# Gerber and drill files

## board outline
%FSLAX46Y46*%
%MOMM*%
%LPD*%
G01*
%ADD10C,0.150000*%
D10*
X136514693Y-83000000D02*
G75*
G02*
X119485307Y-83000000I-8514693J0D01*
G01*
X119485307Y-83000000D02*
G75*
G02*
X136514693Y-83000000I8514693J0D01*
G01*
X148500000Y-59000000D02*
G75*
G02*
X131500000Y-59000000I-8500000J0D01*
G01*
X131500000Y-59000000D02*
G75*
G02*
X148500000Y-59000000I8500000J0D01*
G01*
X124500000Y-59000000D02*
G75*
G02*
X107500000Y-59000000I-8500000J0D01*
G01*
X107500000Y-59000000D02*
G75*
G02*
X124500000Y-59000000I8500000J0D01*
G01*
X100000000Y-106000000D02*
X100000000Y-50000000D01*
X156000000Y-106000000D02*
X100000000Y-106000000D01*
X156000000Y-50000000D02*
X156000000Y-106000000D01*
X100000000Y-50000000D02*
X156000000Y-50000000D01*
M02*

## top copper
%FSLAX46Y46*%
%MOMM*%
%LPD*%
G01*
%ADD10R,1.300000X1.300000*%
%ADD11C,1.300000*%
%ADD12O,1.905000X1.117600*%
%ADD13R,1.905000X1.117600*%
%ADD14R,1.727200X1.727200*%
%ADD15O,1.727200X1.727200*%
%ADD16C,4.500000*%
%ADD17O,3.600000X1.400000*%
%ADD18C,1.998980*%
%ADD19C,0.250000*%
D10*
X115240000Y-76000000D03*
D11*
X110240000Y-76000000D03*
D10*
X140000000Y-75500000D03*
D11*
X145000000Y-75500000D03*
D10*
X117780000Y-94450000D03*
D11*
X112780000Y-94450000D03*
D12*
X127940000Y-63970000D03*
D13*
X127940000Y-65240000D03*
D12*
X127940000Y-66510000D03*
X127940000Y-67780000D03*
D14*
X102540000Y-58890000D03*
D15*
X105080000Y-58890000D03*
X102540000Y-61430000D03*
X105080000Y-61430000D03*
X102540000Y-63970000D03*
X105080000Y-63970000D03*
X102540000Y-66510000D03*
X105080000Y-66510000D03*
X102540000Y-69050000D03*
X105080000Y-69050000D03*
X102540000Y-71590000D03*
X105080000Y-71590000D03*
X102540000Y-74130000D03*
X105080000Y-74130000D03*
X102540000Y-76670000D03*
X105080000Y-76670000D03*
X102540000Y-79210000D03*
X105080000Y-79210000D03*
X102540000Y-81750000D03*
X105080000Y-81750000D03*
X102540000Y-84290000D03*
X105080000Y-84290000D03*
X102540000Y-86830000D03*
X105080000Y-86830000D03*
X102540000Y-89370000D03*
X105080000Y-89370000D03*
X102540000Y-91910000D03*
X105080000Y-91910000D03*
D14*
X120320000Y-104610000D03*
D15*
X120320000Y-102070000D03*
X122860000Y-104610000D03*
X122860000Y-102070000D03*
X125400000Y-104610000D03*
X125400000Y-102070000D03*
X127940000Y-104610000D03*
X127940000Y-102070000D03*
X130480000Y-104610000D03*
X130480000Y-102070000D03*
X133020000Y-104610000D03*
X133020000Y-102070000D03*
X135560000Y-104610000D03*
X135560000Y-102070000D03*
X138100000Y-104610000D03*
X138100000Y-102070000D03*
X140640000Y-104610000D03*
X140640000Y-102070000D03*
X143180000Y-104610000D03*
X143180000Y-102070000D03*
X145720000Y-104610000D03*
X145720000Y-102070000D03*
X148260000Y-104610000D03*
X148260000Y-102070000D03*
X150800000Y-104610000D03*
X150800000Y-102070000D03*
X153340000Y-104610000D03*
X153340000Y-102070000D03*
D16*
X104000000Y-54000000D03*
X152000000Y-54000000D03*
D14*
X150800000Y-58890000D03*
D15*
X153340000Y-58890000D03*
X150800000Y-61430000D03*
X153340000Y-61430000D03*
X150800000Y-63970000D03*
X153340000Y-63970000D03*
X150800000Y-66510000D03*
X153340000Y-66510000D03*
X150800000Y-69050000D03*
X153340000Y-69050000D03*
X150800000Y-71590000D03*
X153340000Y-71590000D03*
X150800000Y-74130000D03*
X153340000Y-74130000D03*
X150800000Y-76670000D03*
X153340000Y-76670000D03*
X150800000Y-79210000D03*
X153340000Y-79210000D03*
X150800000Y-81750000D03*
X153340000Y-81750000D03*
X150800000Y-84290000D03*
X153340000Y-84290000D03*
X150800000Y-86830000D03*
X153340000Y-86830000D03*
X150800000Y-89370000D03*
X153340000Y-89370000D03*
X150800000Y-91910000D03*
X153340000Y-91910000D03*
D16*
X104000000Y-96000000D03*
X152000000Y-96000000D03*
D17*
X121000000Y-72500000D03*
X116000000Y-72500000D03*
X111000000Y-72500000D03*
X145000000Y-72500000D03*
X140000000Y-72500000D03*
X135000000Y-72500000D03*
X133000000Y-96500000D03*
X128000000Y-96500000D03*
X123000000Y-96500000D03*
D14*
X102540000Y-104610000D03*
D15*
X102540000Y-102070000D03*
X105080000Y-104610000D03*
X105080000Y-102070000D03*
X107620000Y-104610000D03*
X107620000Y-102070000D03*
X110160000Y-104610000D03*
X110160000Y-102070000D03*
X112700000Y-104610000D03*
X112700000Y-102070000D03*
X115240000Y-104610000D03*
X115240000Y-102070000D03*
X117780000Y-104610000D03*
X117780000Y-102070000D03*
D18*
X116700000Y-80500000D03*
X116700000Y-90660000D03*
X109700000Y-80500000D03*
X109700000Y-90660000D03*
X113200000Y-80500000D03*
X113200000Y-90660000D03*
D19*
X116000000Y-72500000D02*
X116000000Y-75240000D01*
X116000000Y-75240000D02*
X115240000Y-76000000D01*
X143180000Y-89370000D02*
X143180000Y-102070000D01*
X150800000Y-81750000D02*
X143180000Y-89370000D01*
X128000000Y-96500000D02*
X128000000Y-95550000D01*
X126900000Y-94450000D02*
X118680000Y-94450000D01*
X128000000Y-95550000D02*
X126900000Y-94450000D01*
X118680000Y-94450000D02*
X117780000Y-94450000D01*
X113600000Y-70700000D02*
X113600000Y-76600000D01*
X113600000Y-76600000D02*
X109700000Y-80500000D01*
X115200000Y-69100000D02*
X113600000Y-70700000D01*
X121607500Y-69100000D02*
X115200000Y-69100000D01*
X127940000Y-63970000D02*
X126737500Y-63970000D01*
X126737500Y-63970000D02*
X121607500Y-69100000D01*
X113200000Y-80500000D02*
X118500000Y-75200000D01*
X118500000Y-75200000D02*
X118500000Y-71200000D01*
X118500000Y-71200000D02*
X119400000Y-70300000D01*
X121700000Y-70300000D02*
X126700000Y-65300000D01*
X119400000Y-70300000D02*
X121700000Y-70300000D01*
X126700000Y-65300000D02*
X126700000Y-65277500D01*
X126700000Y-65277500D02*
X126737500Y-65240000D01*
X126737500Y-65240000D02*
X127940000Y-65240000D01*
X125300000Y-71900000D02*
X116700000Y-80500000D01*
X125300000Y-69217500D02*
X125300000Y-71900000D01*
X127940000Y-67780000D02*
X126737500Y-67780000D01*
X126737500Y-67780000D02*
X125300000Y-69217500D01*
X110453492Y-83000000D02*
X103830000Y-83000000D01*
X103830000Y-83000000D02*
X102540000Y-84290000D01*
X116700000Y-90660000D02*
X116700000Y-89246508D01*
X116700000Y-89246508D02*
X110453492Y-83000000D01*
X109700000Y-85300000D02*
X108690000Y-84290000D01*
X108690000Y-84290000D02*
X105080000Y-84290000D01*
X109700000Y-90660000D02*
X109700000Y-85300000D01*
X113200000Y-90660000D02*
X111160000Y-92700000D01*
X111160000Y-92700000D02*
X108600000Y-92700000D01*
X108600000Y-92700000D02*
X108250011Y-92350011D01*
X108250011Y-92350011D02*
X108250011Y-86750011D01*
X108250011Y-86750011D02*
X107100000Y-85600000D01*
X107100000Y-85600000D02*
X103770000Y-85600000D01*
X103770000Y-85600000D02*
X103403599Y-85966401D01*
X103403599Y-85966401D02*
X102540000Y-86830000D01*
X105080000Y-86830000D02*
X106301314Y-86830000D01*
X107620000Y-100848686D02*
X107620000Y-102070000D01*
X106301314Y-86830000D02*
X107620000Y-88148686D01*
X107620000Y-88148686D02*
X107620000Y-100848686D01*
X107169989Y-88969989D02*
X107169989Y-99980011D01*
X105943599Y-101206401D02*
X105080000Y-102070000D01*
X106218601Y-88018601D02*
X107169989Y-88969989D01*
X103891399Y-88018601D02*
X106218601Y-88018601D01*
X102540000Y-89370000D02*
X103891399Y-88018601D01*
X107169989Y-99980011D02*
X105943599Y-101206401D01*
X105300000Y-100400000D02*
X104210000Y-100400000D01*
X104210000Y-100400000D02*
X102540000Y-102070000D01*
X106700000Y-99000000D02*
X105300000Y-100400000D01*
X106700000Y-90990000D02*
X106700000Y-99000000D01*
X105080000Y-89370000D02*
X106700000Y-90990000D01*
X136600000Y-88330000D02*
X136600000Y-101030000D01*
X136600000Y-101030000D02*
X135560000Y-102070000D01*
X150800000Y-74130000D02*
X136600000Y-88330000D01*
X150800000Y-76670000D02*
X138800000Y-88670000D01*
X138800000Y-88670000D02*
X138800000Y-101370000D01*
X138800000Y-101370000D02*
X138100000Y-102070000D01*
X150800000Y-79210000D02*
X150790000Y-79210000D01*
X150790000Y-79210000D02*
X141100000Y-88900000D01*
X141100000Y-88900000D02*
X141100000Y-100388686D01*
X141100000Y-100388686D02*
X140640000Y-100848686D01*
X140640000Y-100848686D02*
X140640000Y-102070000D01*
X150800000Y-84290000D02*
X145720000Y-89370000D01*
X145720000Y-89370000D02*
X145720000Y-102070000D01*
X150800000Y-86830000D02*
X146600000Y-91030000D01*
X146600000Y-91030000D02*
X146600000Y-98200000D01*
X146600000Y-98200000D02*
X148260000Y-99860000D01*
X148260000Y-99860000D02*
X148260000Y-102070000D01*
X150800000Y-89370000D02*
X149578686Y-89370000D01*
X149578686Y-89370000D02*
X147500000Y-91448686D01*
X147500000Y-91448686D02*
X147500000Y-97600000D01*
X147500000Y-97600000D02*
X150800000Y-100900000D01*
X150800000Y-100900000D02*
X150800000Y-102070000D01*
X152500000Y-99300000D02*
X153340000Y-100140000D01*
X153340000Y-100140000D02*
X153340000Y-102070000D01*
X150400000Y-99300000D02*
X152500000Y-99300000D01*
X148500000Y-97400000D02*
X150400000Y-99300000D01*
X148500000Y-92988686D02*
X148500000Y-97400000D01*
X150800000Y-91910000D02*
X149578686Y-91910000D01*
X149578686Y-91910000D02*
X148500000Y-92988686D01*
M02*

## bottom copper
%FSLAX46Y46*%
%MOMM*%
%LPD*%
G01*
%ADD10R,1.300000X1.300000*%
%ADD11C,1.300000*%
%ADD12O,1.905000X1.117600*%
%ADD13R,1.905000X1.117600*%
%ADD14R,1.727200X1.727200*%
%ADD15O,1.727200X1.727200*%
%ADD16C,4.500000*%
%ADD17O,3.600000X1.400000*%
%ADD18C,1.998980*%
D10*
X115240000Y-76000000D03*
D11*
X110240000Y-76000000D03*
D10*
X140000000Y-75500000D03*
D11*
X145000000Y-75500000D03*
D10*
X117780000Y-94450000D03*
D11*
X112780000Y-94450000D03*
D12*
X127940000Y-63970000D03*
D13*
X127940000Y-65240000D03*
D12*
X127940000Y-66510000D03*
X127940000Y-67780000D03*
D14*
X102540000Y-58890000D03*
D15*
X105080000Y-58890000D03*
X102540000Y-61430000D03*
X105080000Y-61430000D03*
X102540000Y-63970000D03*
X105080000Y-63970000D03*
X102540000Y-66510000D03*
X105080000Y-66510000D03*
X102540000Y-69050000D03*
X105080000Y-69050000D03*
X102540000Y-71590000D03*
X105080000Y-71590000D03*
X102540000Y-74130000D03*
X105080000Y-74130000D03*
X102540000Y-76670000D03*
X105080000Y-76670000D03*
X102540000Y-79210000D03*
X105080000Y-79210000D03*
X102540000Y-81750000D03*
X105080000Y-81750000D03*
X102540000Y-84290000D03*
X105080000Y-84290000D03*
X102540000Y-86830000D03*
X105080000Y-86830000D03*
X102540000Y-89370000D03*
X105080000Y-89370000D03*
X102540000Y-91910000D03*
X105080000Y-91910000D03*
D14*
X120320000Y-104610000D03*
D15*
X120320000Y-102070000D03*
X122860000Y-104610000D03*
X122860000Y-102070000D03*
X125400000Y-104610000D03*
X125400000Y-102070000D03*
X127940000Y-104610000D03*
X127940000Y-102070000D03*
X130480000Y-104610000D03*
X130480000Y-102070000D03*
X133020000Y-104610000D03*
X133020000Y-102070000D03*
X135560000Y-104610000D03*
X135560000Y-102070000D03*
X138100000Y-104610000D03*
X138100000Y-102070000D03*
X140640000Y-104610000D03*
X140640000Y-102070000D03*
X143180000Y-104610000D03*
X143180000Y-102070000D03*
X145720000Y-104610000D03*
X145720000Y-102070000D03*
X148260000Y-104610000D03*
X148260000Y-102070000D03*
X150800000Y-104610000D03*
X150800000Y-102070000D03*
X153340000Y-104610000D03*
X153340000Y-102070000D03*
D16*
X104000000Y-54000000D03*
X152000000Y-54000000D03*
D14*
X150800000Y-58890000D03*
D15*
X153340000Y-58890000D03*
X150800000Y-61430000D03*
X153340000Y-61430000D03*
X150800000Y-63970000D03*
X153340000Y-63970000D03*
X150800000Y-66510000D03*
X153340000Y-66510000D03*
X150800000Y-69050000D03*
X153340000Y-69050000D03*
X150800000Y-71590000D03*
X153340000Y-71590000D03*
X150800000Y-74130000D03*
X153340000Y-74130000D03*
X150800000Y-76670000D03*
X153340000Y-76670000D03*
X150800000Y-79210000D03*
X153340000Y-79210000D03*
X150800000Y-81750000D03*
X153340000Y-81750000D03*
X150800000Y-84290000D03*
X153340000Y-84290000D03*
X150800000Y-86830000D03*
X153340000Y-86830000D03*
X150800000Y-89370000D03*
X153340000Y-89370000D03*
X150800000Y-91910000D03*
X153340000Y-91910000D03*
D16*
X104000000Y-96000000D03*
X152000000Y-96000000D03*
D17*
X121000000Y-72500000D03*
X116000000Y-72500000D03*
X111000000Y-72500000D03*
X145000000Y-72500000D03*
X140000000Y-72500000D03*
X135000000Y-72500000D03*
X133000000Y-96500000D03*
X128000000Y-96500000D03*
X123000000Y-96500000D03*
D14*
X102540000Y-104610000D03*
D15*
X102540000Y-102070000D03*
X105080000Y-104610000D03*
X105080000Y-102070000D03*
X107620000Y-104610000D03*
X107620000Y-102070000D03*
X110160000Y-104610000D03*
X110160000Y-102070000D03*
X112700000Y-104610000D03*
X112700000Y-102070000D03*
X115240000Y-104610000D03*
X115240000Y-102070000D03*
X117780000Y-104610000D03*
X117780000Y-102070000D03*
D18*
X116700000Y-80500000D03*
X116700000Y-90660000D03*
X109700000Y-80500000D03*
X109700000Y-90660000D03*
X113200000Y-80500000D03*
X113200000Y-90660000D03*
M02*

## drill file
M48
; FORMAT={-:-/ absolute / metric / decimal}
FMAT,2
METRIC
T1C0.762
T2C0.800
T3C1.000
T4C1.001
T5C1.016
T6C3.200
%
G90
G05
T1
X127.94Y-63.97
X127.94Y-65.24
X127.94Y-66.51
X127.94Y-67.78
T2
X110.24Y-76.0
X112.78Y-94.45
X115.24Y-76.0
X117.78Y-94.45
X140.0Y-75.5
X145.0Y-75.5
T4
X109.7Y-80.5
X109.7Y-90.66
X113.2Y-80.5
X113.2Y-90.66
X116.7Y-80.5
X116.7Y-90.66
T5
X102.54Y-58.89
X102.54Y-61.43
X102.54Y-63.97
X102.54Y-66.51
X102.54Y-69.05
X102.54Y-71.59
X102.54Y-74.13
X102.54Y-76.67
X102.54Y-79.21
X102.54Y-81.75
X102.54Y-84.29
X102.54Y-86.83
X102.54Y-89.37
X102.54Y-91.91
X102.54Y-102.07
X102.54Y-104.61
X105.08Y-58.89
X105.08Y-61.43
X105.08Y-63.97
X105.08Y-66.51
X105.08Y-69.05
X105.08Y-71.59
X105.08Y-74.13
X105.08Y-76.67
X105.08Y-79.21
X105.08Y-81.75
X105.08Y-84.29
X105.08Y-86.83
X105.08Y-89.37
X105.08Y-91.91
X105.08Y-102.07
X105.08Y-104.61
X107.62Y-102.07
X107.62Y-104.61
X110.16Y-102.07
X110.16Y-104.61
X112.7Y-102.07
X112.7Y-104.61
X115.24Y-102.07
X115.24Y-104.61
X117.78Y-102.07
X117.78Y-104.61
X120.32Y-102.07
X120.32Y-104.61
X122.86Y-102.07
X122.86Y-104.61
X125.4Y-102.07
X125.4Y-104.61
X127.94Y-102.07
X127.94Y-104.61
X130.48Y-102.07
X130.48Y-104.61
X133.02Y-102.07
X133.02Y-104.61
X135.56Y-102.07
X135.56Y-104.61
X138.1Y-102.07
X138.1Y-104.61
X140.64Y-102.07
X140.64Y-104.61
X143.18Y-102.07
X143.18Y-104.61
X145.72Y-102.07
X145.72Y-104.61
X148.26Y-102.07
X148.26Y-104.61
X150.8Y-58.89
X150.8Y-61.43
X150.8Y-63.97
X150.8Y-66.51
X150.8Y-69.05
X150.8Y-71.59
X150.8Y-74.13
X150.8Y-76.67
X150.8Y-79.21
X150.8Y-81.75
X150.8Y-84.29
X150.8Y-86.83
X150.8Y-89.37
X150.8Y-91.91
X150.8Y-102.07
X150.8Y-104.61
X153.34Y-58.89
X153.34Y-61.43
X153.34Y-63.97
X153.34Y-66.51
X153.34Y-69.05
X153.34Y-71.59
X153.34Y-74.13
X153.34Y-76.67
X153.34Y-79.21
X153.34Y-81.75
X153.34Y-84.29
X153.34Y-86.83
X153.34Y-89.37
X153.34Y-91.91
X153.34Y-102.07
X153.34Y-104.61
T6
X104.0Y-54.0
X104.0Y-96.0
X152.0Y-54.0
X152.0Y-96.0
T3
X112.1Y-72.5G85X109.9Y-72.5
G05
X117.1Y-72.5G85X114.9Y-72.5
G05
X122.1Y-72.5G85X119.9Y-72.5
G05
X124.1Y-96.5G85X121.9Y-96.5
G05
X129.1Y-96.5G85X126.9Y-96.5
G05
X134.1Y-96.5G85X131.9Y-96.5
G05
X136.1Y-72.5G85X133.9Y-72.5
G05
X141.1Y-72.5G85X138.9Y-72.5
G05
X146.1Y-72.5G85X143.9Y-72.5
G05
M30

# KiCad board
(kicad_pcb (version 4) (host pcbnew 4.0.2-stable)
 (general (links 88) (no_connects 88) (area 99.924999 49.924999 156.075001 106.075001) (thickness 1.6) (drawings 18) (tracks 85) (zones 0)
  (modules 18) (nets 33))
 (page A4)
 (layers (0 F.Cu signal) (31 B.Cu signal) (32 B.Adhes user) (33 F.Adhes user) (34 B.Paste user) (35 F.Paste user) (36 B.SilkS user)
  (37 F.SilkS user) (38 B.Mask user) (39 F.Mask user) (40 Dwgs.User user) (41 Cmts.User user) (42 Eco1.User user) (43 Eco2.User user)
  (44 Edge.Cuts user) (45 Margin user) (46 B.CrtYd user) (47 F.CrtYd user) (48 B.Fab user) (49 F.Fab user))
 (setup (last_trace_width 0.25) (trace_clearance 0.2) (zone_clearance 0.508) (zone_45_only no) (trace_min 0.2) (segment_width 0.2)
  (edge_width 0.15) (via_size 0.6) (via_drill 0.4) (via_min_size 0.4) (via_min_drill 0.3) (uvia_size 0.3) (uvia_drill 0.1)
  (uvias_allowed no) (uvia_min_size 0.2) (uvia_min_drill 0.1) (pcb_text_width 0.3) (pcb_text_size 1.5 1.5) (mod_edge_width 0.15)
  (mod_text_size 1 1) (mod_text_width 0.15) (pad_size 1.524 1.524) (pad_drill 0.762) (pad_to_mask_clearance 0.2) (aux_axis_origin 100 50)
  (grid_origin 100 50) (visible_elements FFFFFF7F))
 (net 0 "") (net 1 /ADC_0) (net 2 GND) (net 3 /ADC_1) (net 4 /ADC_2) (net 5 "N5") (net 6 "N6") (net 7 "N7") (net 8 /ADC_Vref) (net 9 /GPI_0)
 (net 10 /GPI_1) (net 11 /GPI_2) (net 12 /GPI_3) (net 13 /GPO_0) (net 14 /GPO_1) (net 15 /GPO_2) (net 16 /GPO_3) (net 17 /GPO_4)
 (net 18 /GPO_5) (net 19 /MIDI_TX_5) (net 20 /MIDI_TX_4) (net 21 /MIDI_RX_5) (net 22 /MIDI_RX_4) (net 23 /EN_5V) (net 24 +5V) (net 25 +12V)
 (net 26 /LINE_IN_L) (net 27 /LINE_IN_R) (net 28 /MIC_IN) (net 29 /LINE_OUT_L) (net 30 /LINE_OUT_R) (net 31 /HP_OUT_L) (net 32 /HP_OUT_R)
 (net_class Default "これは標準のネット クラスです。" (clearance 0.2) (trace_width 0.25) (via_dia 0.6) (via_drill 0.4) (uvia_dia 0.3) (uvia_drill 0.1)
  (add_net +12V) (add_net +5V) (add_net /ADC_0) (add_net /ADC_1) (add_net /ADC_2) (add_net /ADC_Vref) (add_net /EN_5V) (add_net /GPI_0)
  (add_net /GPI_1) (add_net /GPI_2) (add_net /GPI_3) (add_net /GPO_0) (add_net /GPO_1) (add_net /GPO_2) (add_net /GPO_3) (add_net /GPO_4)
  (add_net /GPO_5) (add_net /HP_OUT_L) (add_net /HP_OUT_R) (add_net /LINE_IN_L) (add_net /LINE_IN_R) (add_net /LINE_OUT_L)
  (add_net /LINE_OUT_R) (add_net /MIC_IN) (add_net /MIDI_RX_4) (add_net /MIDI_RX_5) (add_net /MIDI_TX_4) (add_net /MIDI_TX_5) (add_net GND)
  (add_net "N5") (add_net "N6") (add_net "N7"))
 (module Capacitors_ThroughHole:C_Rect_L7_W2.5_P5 (layer F.Cu) (at 115.24 76 180)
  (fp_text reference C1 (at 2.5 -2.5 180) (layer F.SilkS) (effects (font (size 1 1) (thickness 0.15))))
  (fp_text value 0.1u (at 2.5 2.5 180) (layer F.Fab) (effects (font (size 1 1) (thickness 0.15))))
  (pad 1 thru_hole rect (at 0 0 180) (size 1.3 1.3) (drill 0.8) (layers *.Cu *.Mask) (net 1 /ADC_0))
  (pad 2 thru_hole circle (at 5 0 180) (size 1.3 1.3) (drill 0.8) (layers *.Cu *.Mask) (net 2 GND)))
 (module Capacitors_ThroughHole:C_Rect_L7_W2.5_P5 (layer F.Cu) (at 140 75.5)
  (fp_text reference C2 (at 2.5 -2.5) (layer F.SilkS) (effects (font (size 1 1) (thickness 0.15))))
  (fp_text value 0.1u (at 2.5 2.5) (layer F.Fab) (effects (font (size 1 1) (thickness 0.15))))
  (pad 1 thru_hole rect (at 0 0) (size 1.3 1.3) (drill 0.8) (layers *.Cu *.Mask) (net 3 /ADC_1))
  (pad 2 thru_hole circle (at 5 0) (size 1.3 1.3) (drill 0.8) (layers *.Cu *.Mask) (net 2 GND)))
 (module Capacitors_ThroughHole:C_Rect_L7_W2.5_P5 (layer F.Cu) (at 117.78 94.45 180)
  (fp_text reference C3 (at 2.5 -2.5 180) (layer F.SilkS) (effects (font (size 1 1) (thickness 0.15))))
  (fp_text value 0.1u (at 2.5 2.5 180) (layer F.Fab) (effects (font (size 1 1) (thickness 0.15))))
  (pad 1 thru_hole rect (at 0 0 180) (size 1.3 1.3) (drill 0.8) (layers *.Cu *.Mask) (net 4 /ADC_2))
  (pad 2 thru_hole circle (at 5 0 180) (size 1.3 1.3) (drill 0.8) (layers *.Cu *.Mask) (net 2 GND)))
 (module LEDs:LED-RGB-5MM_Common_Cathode (layer B.Cu) (at 127.94 63.97 180)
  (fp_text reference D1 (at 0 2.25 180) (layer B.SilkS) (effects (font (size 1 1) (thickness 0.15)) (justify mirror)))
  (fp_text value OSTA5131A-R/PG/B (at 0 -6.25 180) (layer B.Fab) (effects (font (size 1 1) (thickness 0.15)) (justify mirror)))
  (pad 1 thru_hole oval (at 0 0 180) (size 1.905 1.1176) (drill 0.762) (layers *.Cu *.Mask) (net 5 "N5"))
  (pad 2 thru_hole rect (at 0 -1.27 180) (size 1.905 1.1176) (drill 0.762) (layers *.Cu *.Mask) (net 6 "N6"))
  (pad 3 thru_hole oval (at 0 -2.54 180) (size 1.905 1.1176) (drill 0.762) (layers *.Cu *.Mask) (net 2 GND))
  (pad 4 thru_hole oval (at 0 -3.81 180) (size 1.905 1.1176) (drill 0.762) (layers *.Cu *.Mask) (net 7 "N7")))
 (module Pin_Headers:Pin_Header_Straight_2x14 (layer F.Cu) (at 102.54 58.89)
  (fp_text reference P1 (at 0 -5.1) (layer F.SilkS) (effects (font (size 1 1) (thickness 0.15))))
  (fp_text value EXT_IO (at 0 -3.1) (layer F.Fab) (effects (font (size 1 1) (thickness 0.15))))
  (pad 1 thru_hole rect (at 0 0) (size 1.7272 1.7272) (drill 1.016) (layers *.Cu *.Mask) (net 1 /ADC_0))
  (pad 2 thru_hole oval (at 2.54 0) (size 1.7272 1.7272) (drill 1.016) (layers *.Cu *.Mask) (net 3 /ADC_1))
  (pad 3 thru_hole oval (at 0 2.54) (size 1.7272 1.7272) (drill 1.016) (layers *.Cu *.Mask) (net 4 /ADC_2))
  (pad 4 thru_hole oval (at 2.54 2.54) (size 1.7272 1.7272) (drill 1.016) (layers *.Cu *.Mask) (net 2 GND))
  (pad 5 thru_hole oval (at 0 5.08) (size 1.7272 1.7272) (drill 1.016) (layers *.Cu *.Mask) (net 2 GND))
  (pad 6 thru_hole oval (at 2.54 5.08) (size 1.7272 1.7272) (drill 1.016) (layers *.Cu *.Mask) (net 2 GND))
  (pad 7 thru_hole oval (at 0 7.62) (size 1.7272 1.7272) (drill 1.016) (layers *.Cu *.Mask) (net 2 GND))
  (pad 8 thru_hole oval (at 2.54 7.62) (size 1.7272 1.7272) (drill 1.016) (layers *.Cu *.Mask) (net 2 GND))
  (pad 9 thru_hole oval (at 0 10.16) (size 1.7272 1.7272) (drill 1.016) (layers *.Cu *.Mask))
  (pad 10 thru_hole oval (at 2.54 10.16) (size 1.7272 1.7272) (drill 1.016) (layers *.Cu *.Mask) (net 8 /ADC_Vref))
  (pad 11 thru_hole oval (at 0 12.7) (size 1.7272 1.7272) (drill 1.016) (layers *.Cu *.Mask) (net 2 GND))
  (pad 12 thru_hole oval (at 2.54 12.7) (size 1.7272 1.7272) (drill 1.016) (layers *.Cu *.Mask) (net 2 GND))
  (pad 13 thru_hole oval (at 0 15.24) (size 1.7272 1.7272) (drill 1.016) (layers *.Cu *.Mask) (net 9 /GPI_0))
  (pad 14 thru_hole oval (at 2.54 15.24) (size 1.7272 1.7272) (drill 1.016) (layers *.Cu *.Mask) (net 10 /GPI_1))
  (pad 15 thru_hole oval (at 0 17.78) (size 1.7272 1.7272) (drill 1.016) (layers *.Cu *.Mask) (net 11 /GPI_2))
  (pad 16 thru_hole oval (at 2.54 17.78) (size 1.7272 1.7272) (drill 1.016) (layers *.Cu *.Mask) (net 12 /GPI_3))
  (pad 17 thru_hole oval (at 0 20.32) (size 1.7272 1.7272) (drill 1.016) (layers *.Cu *.Mask))
  (pad 18 thru_hole oval (at 2.54 20.32) (size 1.7272 1.7272) (drill 1.016) (layers *.Cu *.Mask))
  (pad 19 thru_hole oval (at 0 22.86) (size 1.7272 1.7272) (drill 1.016) (layers *.Cu *.Mask))
  (pad 20 thru_hole oval (at 2.54 22.86) (size 1.7272 1.7272) (drill 1.016) (layers *.Cu *.Mask))
  (pad 21 thru_hole oval (at 0 25.4) (size 1.7272 1.7272) (drill 1.016) (layers *.Cu *.Mask) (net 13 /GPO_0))
  (pad 22 thru_hole oval (at 2.54 25.4) (size 1.7272 1.7272) (drill 1.016) (layers *.Cu *.Mask) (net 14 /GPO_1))
  (pad 23 thru_hole oval (at 0 27.94) (size 1.7272 1.7272) (drill 1.016) (layers *.Cu *.Mask) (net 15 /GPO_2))
  (pad 24 thru_hole oval (at 2.54 27.94) (size 1.7272 1.7272) (drill 1.016) (layers *.Cu *.Mask) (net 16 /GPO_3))
  (pad 25 thru_hole oval (at 0 30.48) (size 1.7272 1.7272) (drill 1.016) (layers *.Cu *.Mask) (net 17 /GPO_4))
  (pad 26 thru_hole oval (at 2.54 30.48) (size 1.7272 1.7272) (drill 1.016) (layers *.Cu *.Mask) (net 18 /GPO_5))
  (pad 27 thru_hole oval (at 0 33.02) (size 1.7272 1.7272) (drill 1.016) (layers *.Cu *.Mask))
  (pad 28 thru_hole oval (at 2.54 33.02) (size 1.7272 1.7272) (drill 1.016) (layers *.Cu *.Mask)))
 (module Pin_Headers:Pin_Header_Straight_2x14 (layer F.Cu) (at 120.32 104.61 90)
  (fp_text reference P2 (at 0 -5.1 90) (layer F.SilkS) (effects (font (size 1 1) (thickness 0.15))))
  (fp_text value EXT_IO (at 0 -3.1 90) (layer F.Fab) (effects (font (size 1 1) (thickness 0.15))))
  (pad 1 thru_hole rect (at 0 0 90) (size 1.7272 1.7272) (drill 1.016) (layers *.Cu *.Mask) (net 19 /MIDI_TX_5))
  (pad 2 thru_hole oval (at 2.54 0 90) (size 1.7272 1.7272) (drill 1.016) (layers *.Cu *.Mask) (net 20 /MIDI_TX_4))
  (pad 3 thru_hole oval (at 0 2.54 90) (size 1.7272 1.7272) (drill 1.016) (layers *.Cu *.Mask) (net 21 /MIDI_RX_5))
  (pad 4 thru_hole oval (at 2.54 2.54 90) (size 1.7272 1.7272) (drill 1.016) (layers *.Cu *.Mask) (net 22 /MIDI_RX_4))
  (pad 5 thru_hole oval (at 0 5.08 90) (size 1.7272 1.7272) (drill 1.016) (layers *.Cu *.Mask) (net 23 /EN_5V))
  (pad 6 thru_hole oval (at 2.54 5.08 90) (size 1.7272 1.7272) (drill 1.016) (layers *.Cu *.Mask) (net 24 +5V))
  (pad 7 thru_hole oval (at 0 7.62 90) (size 1.7272 1.7272) (drill 1.016) (layers *.Cu *.Mask) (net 2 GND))
  (pad 8 thru_hole oval (at 2.54 7.62 90) (size 1.7272 1.7272) (drill 1.016) (layers *.Cu *.Mask) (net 2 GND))
  (pad 9 thru_hole oval (at 0 10.16 90) (size 1.7272 1.7272) (drill 1.016) (layers *.Cu *.Mask) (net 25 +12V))
  (pad 10 thru_hole oval (at 2.54 10.16 90) (size 1.7272 1.7272) (drill 1.016) (layers *.Cu *.Mask) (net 25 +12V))
  (pad 11 thru_hole oval (at 0 12.7 90) (size 1.7272 1.7272) (drill 1.016) (layers *.Cu *.Mask) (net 2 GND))
  (pad 12 thru_hole oval (at 2.54 12.7 90) (size 1.7272 1.7272) (drill 1.016) (layers *.Cu *.Mask) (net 2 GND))
  (pad 13 thru_hole oval (at 0 15.24 90) (size 1.7272 1.7272) (drill 1.016) (layers *.Cu *.Mask) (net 2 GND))
  (pad 14 thru_hole oval (at 2.54 15.24 90) (size 1.7272 1.7272) (drill 1.016) (layers *.Cu *.Mask) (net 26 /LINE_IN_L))
  (pad 15 thru_hole oval (at 0 17.78 90) (size 1.7272 1.7272) (drill 1.016) (layers *.Cu *.Mask) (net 2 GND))
  (pad 16 thru_hole oval (at 2.54 17.78 90) (size 1.7272 1.7272) (drill 1.016) (layers *.Cu *.Mask) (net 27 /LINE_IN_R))
  (pad 17 thru_hole oval (at 0 20.32 90) (size 1.7272 1.7272) (drill 1.016) (layers *.Cu *.Mask) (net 2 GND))
  (pad 18 thru_hole oval (at 2.54 20.32 90) (size 1.7272 1.7272) (drill 1.016) (layers *.Cu *.Mask) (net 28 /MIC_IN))
  (pad 19 thru_hole oval (at 0 22.86 90) (size 1.7272 1.7272) (drill 1.016) (layers *.Cu *.Mask) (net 2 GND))
  (pad 20 thru_hole oval (at 2.54 22.86 90) (size 1.7272 1.7272) (drill 1.016) (layers *.Cu *.Mask) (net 2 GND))
  (pad 21 thru_hole oval (at 0 25.4 90) (size 1.7272 1.7272) (drill 1.016) (layers *.Cu *.Mask) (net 2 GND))
  (pad 22 thru_hole oval (at 2.54 25.4 90) (size 1.7272 1.7272) (drill 1.016) (layers *.Cu *.Mask) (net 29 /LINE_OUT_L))
  (pad 23 thru_hole oval (at 0 27.94 90) (size 1.7272 1.7272) (drill 1.016) (layers *.Cu *.Mask) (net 2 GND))
  (pad 24 thru_hole oval (at 2.54 27.94 90) (size 1.7272 1.7272) (drill 1.016) (layers *.Cu *.Mask) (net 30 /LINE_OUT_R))
  (pad 25 thru_hole oval (at 0 30.48 90) (size 1.7272 1.7272) (drill 1.016) (layers *.Cu *.Mask) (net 2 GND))
  (pad 26 thru_hole oval (at 2.54 30.48 90) (size 1.7272 1.7272) (drill 1.016) (layers *.Cu *.Mask) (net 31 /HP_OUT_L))
  (pad 27 thru_hole oval (at 0 33.02 90) (size 1.7272 1.7272) (drill 1.016) (layers *.Cu *.Mask) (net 2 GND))
  (pad 28 thru_hole oval (at 2.54 33.02 90) (size 1.7272 1.7272) (drill 1.016) (layers *.Cu *.Mask) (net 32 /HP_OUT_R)))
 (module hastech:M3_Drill (layer F.Cu) (at 104 54)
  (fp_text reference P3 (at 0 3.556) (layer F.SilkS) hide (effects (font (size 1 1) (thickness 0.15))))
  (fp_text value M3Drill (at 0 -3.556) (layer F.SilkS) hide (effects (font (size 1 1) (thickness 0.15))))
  (pad 1 thru_hole circle (at 0 0) (size 4.5 4.5) (drill 3.2) (layers *.Cu *.Mask F.SilkS) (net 2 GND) (zone_connect 2)))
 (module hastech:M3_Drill (layer F.Cu) (at 152 54)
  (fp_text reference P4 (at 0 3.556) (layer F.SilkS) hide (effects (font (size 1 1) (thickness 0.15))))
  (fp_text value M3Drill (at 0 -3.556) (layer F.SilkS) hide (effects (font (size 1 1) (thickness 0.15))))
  (pad 1 thru_hole circle (at 0 0) (size 4.5 4.5) (drill 3.2) (layers *.Cu *.Mask F.SilkS) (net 2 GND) (zone_connect 2)))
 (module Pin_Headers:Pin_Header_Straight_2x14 (layer F.Cu) (at 150.8 58.89)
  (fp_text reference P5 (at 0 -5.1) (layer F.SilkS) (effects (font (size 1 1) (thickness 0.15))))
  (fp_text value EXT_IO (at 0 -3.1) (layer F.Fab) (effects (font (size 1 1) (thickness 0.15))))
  (pad 1 thru_hole rect (at 0 0) (size 1.7272 1.7272) (drill 1.016) (layers *.Cu *.Mask) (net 20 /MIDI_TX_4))
  (pad 2 thru_hole oval (at 2.54 0) (size 1.7272 1.7272) (drill 1.016) (layers *.Cu *.Mask) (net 19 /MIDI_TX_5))
  (pad 3 thru_hole oval (at 0 2.54) (size 1.7272 1.7272) (drill 1.016) (layers *.Cu *.Mask) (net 22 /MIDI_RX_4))
  (pad 4 thru_hole oval (at 2.54 2.54) (size 1.7272 1.7272) (drill 1.016) (layers *.Cu *.Mask) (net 21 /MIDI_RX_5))
  (pad 5 thru_hole oval (at 0 5.08) (size 1.7272 1.7272) (drill 1.016) (layers *.Cu *.Mask) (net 24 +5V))
  (pad 6 thru_hole oval (at 2.54 5.08) (size 1.7272 1.7272) (drill 1.016) (layers *.Cu *.Mask) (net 23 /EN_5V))
  (pad 7 thru_hole oval (at 0 7.62) (size 1.7272 1.7272) (drill 1.016) (layers *.Cu *.Mask) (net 2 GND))
  (pad 8 thru_hole oval (at 2.54 7.62) (size 1.7272 1.7272) (drill 1.016) (layers *.Cu *.Mask) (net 2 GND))
  (pad 9 thru_hole oval (at 0 10.16) (size 1.7272 1.7272) (drill 1.016) (layers *.Cu *.Mask) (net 25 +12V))
  (pad 10 thru_hole oval (at 2.54 10.16) (size 1.7272 1.7272) (drill 1.016) (layers *.Cu *.Mask) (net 25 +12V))
  (pad 11 thru_hole oval (at 0 12.7) (size 1.7272 1.7272) (drill 1.016) (layers *.Cu *.Mask) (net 2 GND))
  (pad 12 thru_hole oval (at 2.54 12.7) (size 1.7272 1.7272) (drill 1.016) (layers *.Cu *.Mask) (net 2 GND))
  (pad 13 thru_hole oval (at 0 15.24) (size 1.7272 1.7272) (drill 1.016) (layers *.Cu *.Mask) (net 26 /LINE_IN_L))
  (pad 14 thru_hole oval (at 2.54 15.24) (size 1.7272 1.7272) (drill 1.016) (layers *.Cu *.Mask) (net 2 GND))
  (pad 15 thru_hole oval (at 0 17.78) (size 1.7272 1.7272) (drill 1.016) (layers *.Cu *.Mask) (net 27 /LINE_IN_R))
  (pad 16 thru_hole oval (at 2.54 17.78) (size 1.7272 1.7272) (drill 1.016) (layers *.Cu *.Mask) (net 2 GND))
  (pad 17 thru_hole oval (at 0 20.32) (size 1.7272 1.7272) (drill 1.016) (layers *.Cu *.Mask) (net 28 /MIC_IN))
  (pad 18 thru_hole oval (at 2.54 20.32) (size 1.7272 1.7272) (drill 1.016) (layers *.Cu *.Mask) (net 2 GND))
  (pad 19 thru_hole oval (at 0 22.86) (size 1.7272 1.7272) (drill 1.016) (layers *.Cu *.Mask) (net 2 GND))
  (pad 20 thru_hole oval (at 2.54 22.86) (size 1.7272 1.7272) (drill 1.016) (layers *.Cu *.Mask) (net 2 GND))
  (pad 21 thru_hole oval (at 0 25.4) (size 1.7272 1.7272) (drill 1.016) (layers *.Cu *.Mask) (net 29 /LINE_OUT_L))
  (pad 22 thru_hole oval (at 2.54 25.4) (size 1.7272 1.7272) (drill 1.016) (layers *.Cu *.Mask) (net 2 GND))
  (pad 23 thru_hole oval (at 0 27.94) (size 1.7272 1.7272) (drill 1.016) (layers *.Cu *.Mask) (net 30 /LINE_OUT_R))
  (pad 24 thru_hole oval (at 2.54 27.94) (size 1.7272 1.7272) (drill 1.016) (layers *.Cu *.Mask) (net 2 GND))
  (pad 25 thru_hole oval (at 0 30.48) (size 1.7272 1.7272) (drill 1.016) (layers *.Cu *.Mask) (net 31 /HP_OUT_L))
  (pad 26 thru_hole oval (at 2.54 30.48) (size 1.7272 1.7272) (drill 1.016) (layers *.Cu *.Mask) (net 2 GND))
  (pad 27 thru_hole oval (at 0 33.02) (size 1.7272 1.7272) (drill 1.016) (layers *.Cu *.Mask) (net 32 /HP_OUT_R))
  (pad 28 thru_hole oval (at 2.54 33.02) (size 1.7272 1.7272) (drill 1.016) (layers *.Cu *.Mask) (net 2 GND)))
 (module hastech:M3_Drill (layer F.Cu) (at 104 96)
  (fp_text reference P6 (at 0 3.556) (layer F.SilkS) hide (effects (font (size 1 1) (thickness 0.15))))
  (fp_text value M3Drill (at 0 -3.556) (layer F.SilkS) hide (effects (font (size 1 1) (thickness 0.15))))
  (pad 1 thru_hole circle (at 0 0) (size 4.5 4.5) (drill 3.2) (layers *.Cu *.Mask F.SilkS) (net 2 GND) (zone_connect 2)))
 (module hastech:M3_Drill (layer F.Cu) (at 152 96)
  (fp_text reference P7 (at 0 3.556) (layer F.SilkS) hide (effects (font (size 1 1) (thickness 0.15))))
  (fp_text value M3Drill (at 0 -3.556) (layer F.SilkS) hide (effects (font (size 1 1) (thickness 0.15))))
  (pad 1 thru_hole circle (at 0 0) (size 4.5 4.5) (drill 3.2) (layers *.Cu *.Mask F.SilkS) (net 2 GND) (zone_connect 2)))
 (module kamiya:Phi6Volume (layer B.Cu) (at 116 59 180)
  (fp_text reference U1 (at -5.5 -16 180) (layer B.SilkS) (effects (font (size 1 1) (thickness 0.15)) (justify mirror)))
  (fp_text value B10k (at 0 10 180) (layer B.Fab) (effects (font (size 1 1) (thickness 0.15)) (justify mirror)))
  (pad 1 thru_hole oval (at -5 -13.5 180) (size 3.6 1.4) (drill oval 3.2 1) (layers *.Cu *.Mask B.SilkS) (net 8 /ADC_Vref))
  (pad 2 thru_hole oval (at 0 -13.5 180) (size 3.6 1.4) (drill oval 3.2 1) (layers *.Cu *.Mask B.SilkS) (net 1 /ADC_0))
  (pad 3 thru_hole oval (at 5 -13.5 180) (size 3.6 1.4) (drill oval 3.2 1) (layers *.Cu *.Mask B.SilkS) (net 2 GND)))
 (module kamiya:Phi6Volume (layer B.Cu) (at 140 59 180)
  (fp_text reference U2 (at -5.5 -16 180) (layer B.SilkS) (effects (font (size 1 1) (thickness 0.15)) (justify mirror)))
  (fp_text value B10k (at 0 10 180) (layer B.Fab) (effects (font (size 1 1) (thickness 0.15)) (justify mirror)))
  (pad 1 thru_hole oval (at -5 -13.5 180) (size 3.6 1.4) (drill oval 3.2 1) (layers *.Cu *.Mask B.SilkS) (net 8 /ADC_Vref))
  (pad 2 thru_hole oval (at 0 -13.5 180) (size 3.6 1.4) (drill oval 3.2 1) (layers *.Cu *.Mask B.SilkS) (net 3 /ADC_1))
  (pad 3 thru_hole oval (at 5 -13.5 180) (size 3.6 1.4) (drill oval 3.2 1) (layers *.Cu *.Mask B.SilkS) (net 2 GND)))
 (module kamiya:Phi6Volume (layer B.Cu) (at 128 83 180)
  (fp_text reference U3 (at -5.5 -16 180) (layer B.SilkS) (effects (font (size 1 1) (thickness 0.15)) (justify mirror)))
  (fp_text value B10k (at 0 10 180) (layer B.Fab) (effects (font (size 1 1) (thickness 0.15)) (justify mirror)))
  (pad 1 thru_hole oval (at -5 -13.5 180) (size 3.6 1.4) (drill oval 3.2 1) (layers *.Cu *.Mask B.SilkS) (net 8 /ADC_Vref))
  (pad 2 thru_hole oval (at 0 -13.5 180) (size 3.6 1.4) (drill oval 3.2 1) (layers *.Cu *.Mask B.SilkS) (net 4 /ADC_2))
  (pad 3 thru_hole oval (at 5 -13.5 180) (size 3.6 1.4) (drill oval 3.2 1) (layers *.Cu *.Mask B.SilkS) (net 2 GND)))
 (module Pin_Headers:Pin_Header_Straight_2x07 (layer F.Cu) (at 102.54 104.61 90)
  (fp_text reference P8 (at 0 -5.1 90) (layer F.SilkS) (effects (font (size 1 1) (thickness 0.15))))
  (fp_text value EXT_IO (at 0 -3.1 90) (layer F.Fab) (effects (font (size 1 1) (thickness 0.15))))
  (pad 1 thru_hole rect (at 0 0 90) (size 1.7272 1.7272) (drill 1.016) (layers *.Cu *.Mask) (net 2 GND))
  (pad 2 thru_hole oval (at 2.54 0 90) (size 1.7272 1.7272) (drill 1.016) (layers *.Cu *.Mask) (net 18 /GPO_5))
  (pad 3 thru_hole oval (at 0 2.54 90) (size 1.7272 1.7272) (drill 1.016) (layers *.Cu *.Mask) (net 2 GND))
  (pad 4 thru_hole oval (at 2.54 2.54 90) (size 1.7272 1.7272) (drill 1.016) (layers *.Cu *.Mask) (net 17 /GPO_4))
  (pad 5 thru_hole oval (at 0 5.08 90) (size 1.7272 1.7272) (drill 1.016) (layers *.Cu *.Mask) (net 2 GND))
  (pad 6 thru_hole oval (at 2.54 5.08 90) (size 1.7272 1.7272) (drill 1.016) (layers *.Cu *.Mask) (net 16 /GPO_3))
  (pad 7 thru_hole oval (at 0 7.62 90) (size 1.7272 1.7272) (drill 1.016) (layers *.Cu *.Mask) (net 2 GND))
  (pad 8 thru_hole oval (at 2.54 7.62 90) (size 1.7272 1.7272) (drill 1.016) (layers *.Cu *.Mask) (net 12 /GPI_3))
  (pad 9 thru_hole oval (at 0 10.16 90) (size 1.7272 1.7272) (drill 1.016) (layers *.Cu *.Mask) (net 2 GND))
  (pad 10 thru_hole oval (at 2.54 10.16 90) (size 1.7272 1.7272) (drill 1.016) (layers *.Cu *.Mask) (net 11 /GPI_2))
  (pad 11 thru_hole oval (at 0 12.7 90) (size 1.7272 1.7272) (drill 1.016) (layers *.Cu *.Mask) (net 2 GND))
  (pad 12 thru_hole oval (at 2.54 12.7 90) (size 1.7272 1.7272) (drill 1.016) (layers *.Cu *.Mask) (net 10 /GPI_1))
  (pad 13 thru_hole oval (at 0 15.24 90) (size 1.7272 1.7272) (drill 1.016) (layers *.Cu *.Mask) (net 2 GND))
  (pad 14 thru_hole oval (at 2.54 15.24 90) (size 1.7272 1.7272) (drill 1.016) (layers *.Cu *.Mask) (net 9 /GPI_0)))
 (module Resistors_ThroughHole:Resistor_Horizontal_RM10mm (layer F.Cu) (at 116.7 80.5 270)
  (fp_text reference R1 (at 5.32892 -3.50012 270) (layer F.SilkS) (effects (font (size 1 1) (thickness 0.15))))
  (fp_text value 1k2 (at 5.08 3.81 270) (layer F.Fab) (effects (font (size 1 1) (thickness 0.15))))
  (pad 1 thru_hole circle (at 0 0 270) (size 1.99898 1.99898) (drill 1.00076) (layers *.Cu *.SilkS *.Mask) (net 7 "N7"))
  (pad 2 thru_hole circle (at 10.16 0 270) (size 1.99898 1.99898) (drill 1.00076) (layers *.Cu *.SilkS *.Mask) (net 13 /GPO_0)))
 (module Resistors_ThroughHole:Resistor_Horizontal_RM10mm (layer F.Cu) (at 109.7 80.5 270)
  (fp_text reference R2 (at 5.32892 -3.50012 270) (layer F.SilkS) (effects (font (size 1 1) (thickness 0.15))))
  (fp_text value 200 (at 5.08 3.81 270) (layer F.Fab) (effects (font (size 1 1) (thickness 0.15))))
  (pad 1 thru_hole circle (at 0 0 270) (size 1.99898 1.99898) (drill 1.00076) (layers *.Cu *.SilkS *.Mask) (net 5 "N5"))
  (pad 2 thru_hole circle (at 10.16 0 270) (size 1.99898 1.99898) (drill 1.00076) (layers *.Cu *.SilkS *.Mask) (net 14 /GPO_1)))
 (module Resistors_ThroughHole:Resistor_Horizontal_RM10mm (layer F.Cu) (at 113.2 80.5 270)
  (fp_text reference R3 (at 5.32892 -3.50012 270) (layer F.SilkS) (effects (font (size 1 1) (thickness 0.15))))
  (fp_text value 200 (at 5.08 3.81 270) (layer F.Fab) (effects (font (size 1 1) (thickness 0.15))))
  (pad 1 thru_hole circle (at 0 0 270) (size 1.99898 1.99898) (drill 1.00076) (layers *.Cu *.SilkS *.Mask) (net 6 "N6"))
  (pad 2 thru_hole circle (at 10.16 0 270) (size 1.99898 1.99898) (drill 1.00076) (layers *.Cu *.SilkS *.Mask) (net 15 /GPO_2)))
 (gr_circle (center 128 83) (end 136.5 82.5) (layer Edge.Cuts) (width 0.15))
 (gr_circle (center 140 59) (end 148.5 59) (layer Edge.Cuts) (width 0.15))
 (gr_circle (center 116 59) (end 124.5 59) (layer Edge.Cuts) (width 0.15))
 (gr_line (start 100 106) (end 100 50) (layer Edge.Cuts) (width 0.15))
 (gr_line (start 156 106) (end 100 106) (layer Edge.Cuts) (width 0.15))
 (gr_line (start 156 50) (end 156 106) (layer Edge.Cuts) (width 0.15))
 (gr_line (start 100 50) (end 156 50) (layer Edge.Cuts) (width 0.15))
 (segment (start 116 72.5) (end 116 75.24) (width 0.25) (layer F.Cu) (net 1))
 (segment (start 116 75.24) (end 115.24 76) (width 0.25) (layer F.Cu) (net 1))
 (segment (start 143.18 89.37) (end 143.18 102.07) (width 0.25) (layer F.Cu) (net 2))
 (segment (start 150.8 81.75) (end 143.18 89.37) (width 0.25) (layer F.Cu) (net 2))
 (segment (start 128 96.5) (end 128 95.55) (width 0.25) (layer F.Cu) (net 4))
 (segment (start 126.9 94.45) (end 118.68 94.45) (width 0.25) (layer F.Cu) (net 4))
 (segment (start 128 95.55) (end 126.9 94.45) (width 0.25) (layer F.Cu) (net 4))
 (segment (start 118.68 94.45) (end 117.78 94.45) (width 0.25) (layer F.Cu) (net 4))
 (segment (start 113.6 70.7) (end 113.6 76.6) (width 0.25) (layer F.Cu) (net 5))
 (segment (start 113.6 76.6) (end 109.7 80.5) (width 0.25) (layer F.Cu) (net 5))
 (segment (start 115.2 69.1) (end 113.6 70.7) (width 0.25) (layer F.Cu) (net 5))
 (segment (start 121.6075 69.1) (end 115.2 69.1) (width 0.25) (layer F.Cu) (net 5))
 (segment (start 127.94 63.97) (end 126.7375 63.97) (width 0.25) (layer F.Cu) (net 5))
 (segment (start 126.7375 63.97) (end 121.6075 69.1) (width 0.25) (layer F.Cu) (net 5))
 (segment (start 113.2 80.5) (end 118.5 75.2) (width 0.25) (layer F.Cu) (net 6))
 (segment (start 118.5 75.2) (end 118.5 71.2) (width 0.25) (layer F.Cu) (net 6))
 (segment (start 118.5 71.2) (end 119.4 70.3) (width 0.25) (layer F.Cu) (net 6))
 (segment (start 121.7 70.3) (end 126.7 65.3) (width 0.25) (layer F.Cu) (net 6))
 (segment (start 119.4 70.3) (end 121.7 70.3) (width 0.25) (layer F.Cu) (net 6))
 (segment (start 126.7 65.3) (end 126.7 65.2775) (width 0.25) (layer F.Cu) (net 6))
 (segment (start 126.7 65.2775) (end 126.7375 65.24) (width 0.25) (layer F.Cu) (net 6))
 (segment (start 126.7375 65.24) (end 127.94 65.24) (width 0.25) (layer F.Cu) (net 6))
 (segment (start 125.3 71.9) (end 116.7 80.5) (width 0.25) (layer F.Cu) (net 7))
 (segment (start 125.3 69.2175) (end 125.3 71.9) (width 0.25) (layer F.Cu) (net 7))
 (segment (start 127.94 67.78) (end 126.7375 67.78) (width 0.25) (layer F.Cu) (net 7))
 (segment (start 126.7375 67.78) (end 125.3 69.2175) (width 0.25) (layer F.Cu) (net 7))
 (segment (start 110.453492 83) (end 103.83 83) (width 0.25) (layer F.Cu) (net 13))
 (segment (start 103.83 83) (end 102.54 84.29) (width 0.25) (layer F.Cu) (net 13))
 (segment (start 116.7 90.66) (end 116.7 89.246508) (width 0.25) (layer F.Cu) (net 13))
 (segment (start 116.7 89.246508) (end 110.453492 83) (width 0.25) (layer F.Cu) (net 13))
 (segment (start 109.7 85.3) (end 108.69 84.29) (width 0.25) (layer F.Cu) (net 14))
 (segment (start 108.69 84.29) (end 105.08 84.29) (width 0.25) (layer F.Cu) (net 14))
 (segment (start 109.7 90.66) (end 109.7 85.3) (width 0.25) (layer F.Cu) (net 14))
 (segment (start 113.2 90.66) (end 111.16 92.7) (width 0.25) (layer F.Cu) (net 15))
 (segment (start 111.16 92.7) (end 108.6 92.7) (width 0.25) (layer F.Cu) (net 15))
 (segment (start 108.6 92.7) (end 108.250011 92.350011) (width 0.25) (layer F.Cu) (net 15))
 (segment (start 108.250011 92.350011) (end 108.250011 86.750011) (width 0.25) (layer F.Cu) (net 15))
 (segment (start 108.250011 86.750011) (end 107.1 85.6) (width 0.25) (layer F.Cu) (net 15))
 (segment (start 107.1 85.6) (end 103.77 85.6) (width 0.25) (layer F.Cu) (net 15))
 (segment (start 103.77 85.6) (end 103.403599 85.966401) (width 0.25) (layer F.Cu) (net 15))
 (segment (start 103.403599 85.966401) (end 102.54 86.83) (width 0.25) (layer F.Cu) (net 15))
 (segment (start 105.08 86.83) (end 106.301314 86.83) (width 0.25) (layer F.Cu) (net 16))
 (segment (start 107.62 100.848686) (end 107.62 102.07) (width 0.25) (layer F.Cu) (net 16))
 (segment (start 106.301314 86.83) (end 107.62 88.148686) (width 0.25) (layer F.Cu) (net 16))
 (segment (start 107.62 88.148686) (end 107.62 100.848686) (width 0.25) (layer F.Cu) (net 16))
 (segment (start 107.169989 88.969989) (end 107.169989 99.980011) (width 0.25) (layer F.Cu) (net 17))
 (segment (start 105.943599 101.206401) (end 105.08 102.07) (width 0.25) (layer F.Cu) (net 17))
 (segment (start 106.218601 88.018601) (end 107.169989 88.969989) (width 0.25) (layer F.Cu) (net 17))
 (segment (start 103.891399 88.018601) (end 106.218601 88.018601) (width 0.25) (layer F.Cu) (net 17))
 (segment (start 102.54 89.37) (end 103.891399 88.018601) (width 0.25) (layer F.Cu) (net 17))
 (segment (start 107.169989 99.980011) (end 105.943599 101.206401) (width 0.25) (layer F.Cu) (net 17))
 (segment (start 105.3 100.4) (end 104.21 100.4) (width 0.25) (layer F.Cu) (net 18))
 (segment (start 104.21 100.4) (end 102.54 102.07) (width 0.25) (layer F.Cu) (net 18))
 (segment (start 106.7 99) (end 105.3 100.4) (width 0.25) (layer F.Cu) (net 18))
 (segment (start 106.7 90.99) (end 106.7 99) (width 0.25) (layer F.Cu) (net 18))
 (segment (start 105.08 89.37) (end 106.7 90.99) (width 0.25) (layer F.Cu) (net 18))
 (segment (start 136.6 88.33) (end 136.6 101.03) (width 0.25) (layer F.Cu) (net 26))
 (segment (start 136.6 101.03) (end 135.56 102.07) (width 0.25) (layer F.Cu) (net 26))
 (segment (start 150.8 74.13) (end 136.6 88.33) (width 0.25) (layer F.Cu) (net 26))
 (segment (start 150.8 76.67) (end 138.8 88.67) (width 0.25) (layer F.Cu) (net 27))
 (segment (start 138.8 88.67) (end 138.8 101.37) (width 0.25) (layer F.Cu) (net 27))
 (segment (start 138.8 101.37) (end 138.1 102.07) (width 0.25) (layer F.Cu) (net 27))
 (segment (start 150.8 79.21) (end 150.79 79.21) (width 0.25) (layer F.Cu) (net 28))
 (segment (start 150.79 79.21) (end 141.1 88.9) (width 0.25) (layer F.Cu) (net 28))
 (segment (start 141.1 88.9) (end 141.1 100.388686) (width 0.25) (layer F.Cu) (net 28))
 (segment (start 141.1 100.388686) (end 140.64 100.848686) (width 0.25) (layer F.Cu) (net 28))
 (segment (start 140.64 100.848686) (end 140.64 102.07) (width 0.25) (layer F.Cu) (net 28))
 (segment (start 150.8 84.29) (end 145.72 89.37) (width 0.25) (layer F.Cu) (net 29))
 (segment (start 145.72 89.37) (end 145.72 102.07) (width 0.25) (layer F.Cu) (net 29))
 (segment (start 150.8 86.83) (end 146.6 91.03) (width 0.25) (layer F.Cu) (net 30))
 (segment (start 146.6 91.03) (end 146.6 98.2) (width 0.25) (layer F.Cu) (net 30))
 (segment (start 146.6 98.2) (end 148.26 99.86) (width 0.25) (layer F.Cu) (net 30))
 (segment (start 148.26 99.86) (end 148.26 102.07) (width 0.25) (layer F.Cu) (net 30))
 (segment (start 150.8 89.37) (end 149.578686 89.37) (width 0.25) (layer F.Cu) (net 31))
 (segment (start 149.578686 89.37) (end 147.5 91.448686) (width 0.25) (layer F.Cu) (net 31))
 (segment (start 147.5 91.448686) (end 147.5 97.6) (width 0.25) (layer F.Cu) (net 31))
 (segment (start 147.5 97.6) (end 150.8 100.9) (width 0.25) (layer F.Cu) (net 31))
 (segment (start 150.8 100.9) (end 150.8 102.07) (width 0.25) (layer F.Cu) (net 31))
 (segment (start 152.5 99.3) (end 153.34 100.14) (width 0.25) (layer F.Cu) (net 32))
 (segment (start 153.34 100.14) (end 153.34 102.07) (width 0.25) (layer F.Cu) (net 32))
 (segment (start 150.4 99.3) (end 152.5 99.3) (width 0.25) (layer F.Cu) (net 32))
 (segment (start 148.5 97.4) (end 150.4 99.3) (width 0.25) (layer F.Cu) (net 32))
 (segment (start 148.5 92.988686) (end 148.5 97.4) (width 0.25) (layer F.Cu) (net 32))
 (segment (start 150.8 91.91) (end 149.578686 91.91) (width 0.25) (layer F.Cu) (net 32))
 (segment (start 149.578686 91.91) (end 148.5 92.988686) (width 0.25) (layer F.Cu) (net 32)))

